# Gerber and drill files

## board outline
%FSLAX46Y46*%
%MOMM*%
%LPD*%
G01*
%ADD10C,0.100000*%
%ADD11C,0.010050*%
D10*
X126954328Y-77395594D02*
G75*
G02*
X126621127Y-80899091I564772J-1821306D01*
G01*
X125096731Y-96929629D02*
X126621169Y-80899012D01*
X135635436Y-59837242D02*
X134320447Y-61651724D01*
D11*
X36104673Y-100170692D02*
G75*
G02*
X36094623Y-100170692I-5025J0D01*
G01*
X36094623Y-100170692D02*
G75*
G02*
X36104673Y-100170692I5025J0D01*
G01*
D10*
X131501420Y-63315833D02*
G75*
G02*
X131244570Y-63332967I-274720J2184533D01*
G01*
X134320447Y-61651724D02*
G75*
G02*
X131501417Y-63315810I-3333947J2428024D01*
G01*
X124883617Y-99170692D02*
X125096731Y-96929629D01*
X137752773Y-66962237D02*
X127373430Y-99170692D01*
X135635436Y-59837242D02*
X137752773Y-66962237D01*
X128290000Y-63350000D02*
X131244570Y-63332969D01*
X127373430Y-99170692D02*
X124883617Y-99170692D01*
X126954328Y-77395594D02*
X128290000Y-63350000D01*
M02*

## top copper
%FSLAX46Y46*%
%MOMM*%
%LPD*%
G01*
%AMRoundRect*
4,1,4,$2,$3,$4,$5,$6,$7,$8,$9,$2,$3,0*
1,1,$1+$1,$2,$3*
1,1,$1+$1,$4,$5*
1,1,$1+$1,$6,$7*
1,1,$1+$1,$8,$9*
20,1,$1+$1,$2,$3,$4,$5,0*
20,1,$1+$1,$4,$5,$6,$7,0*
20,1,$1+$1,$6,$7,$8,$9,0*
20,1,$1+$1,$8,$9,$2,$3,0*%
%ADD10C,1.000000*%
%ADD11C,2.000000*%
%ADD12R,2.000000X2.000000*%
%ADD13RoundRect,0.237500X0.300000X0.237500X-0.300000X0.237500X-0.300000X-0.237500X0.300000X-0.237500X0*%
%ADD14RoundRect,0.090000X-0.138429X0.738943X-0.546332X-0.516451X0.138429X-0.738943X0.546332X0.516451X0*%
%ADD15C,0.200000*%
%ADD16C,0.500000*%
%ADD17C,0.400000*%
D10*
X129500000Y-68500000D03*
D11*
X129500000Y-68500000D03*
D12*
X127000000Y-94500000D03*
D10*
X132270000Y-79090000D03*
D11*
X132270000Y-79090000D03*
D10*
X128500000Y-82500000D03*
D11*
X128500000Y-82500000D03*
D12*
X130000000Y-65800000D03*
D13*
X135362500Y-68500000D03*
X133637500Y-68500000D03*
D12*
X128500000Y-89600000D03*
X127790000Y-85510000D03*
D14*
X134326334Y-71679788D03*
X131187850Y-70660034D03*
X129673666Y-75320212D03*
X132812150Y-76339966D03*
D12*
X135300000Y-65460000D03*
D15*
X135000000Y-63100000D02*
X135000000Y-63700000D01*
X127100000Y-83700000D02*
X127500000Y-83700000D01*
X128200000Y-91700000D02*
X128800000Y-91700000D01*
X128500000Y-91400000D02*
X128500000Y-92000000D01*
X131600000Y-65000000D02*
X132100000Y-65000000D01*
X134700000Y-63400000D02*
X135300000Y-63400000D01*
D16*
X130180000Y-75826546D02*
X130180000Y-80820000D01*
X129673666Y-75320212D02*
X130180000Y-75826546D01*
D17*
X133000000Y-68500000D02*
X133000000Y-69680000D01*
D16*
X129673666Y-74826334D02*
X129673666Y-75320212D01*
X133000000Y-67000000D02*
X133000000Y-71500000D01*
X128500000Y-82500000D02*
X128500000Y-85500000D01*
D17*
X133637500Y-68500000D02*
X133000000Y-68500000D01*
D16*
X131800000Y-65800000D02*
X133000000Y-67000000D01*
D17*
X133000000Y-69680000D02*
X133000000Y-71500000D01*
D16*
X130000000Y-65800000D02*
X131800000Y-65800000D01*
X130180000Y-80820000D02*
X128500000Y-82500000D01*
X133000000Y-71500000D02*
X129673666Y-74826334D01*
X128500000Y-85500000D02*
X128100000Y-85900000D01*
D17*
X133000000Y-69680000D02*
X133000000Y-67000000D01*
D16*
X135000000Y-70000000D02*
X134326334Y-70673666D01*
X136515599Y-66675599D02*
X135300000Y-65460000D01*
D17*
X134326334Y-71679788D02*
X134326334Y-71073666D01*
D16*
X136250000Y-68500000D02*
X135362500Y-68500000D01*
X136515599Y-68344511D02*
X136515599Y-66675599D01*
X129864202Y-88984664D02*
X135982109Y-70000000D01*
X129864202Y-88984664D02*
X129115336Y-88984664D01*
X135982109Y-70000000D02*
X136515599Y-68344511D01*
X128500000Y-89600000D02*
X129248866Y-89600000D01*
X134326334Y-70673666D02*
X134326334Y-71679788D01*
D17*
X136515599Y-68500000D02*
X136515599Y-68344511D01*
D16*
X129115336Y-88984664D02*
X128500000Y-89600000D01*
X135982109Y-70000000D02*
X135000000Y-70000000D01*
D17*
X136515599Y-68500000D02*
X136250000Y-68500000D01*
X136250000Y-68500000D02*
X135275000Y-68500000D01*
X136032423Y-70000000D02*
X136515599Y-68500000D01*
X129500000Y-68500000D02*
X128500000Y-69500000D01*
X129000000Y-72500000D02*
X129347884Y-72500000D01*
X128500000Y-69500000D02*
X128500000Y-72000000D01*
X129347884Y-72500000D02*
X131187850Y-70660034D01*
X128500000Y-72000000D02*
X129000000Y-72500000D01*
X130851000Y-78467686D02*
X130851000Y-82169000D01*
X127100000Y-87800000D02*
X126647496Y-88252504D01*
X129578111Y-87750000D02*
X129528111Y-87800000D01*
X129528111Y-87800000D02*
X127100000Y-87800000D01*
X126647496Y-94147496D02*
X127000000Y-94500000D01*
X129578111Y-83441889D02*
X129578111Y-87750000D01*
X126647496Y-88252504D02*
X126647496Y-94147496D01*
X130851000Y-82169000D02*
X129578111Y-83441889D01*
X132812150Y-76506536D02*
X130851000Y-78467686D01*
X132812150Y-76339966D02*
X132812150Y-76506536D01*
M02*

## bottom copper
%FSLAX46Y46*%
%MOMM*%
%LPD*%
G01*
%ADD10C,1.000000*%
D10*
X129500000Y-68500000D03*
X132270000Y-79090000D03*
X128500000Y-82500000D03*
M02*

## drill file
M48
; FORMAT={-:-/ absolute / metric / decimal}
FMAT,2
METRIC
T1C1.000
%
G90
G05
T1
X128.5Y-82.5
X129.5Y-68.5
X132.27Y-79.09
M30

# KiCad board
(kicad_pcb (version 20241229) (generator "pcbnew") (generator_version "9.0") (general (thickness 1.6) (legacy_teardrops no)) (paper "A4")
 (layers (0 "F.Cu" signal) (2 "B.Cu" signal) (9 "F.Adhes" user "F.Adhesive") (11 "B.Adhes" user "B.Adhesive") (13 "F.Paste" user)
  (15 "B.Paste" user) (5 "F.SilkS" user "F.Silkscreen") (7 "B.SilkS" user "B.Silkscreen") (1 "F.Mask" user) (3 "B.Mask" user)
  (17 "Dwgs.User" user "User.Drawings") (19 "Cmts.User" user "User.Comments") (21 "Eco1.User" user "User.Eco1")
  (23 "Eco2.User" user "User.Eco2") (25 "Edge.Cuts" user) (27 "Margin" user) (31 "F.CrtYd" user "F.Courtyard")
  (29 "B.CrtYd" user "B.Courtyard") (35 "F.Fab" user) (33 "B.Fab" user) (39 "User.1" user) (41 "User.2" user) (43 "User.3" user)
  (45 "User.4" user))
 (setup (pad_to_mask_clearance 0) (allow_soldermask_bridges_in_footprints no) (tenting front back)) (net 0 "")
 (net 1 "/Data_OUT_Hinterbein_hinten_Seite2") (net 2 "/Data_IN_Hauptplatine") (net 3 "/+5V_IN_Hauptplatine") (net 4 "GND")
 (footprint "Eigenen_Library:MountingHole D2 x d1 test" (layer "F.Cu") (at 129.5 68.5)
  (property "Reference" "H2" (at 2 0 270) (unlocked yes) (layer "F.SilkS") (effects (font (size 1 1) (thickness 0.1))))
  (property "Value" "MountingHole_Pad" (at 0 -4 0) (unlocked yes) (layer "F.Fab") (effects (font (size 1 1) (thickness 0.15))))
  (pad "1" thru_hole circle (at 0 0) (size 1 1) (drill 1) (layers "*.Cu" "*.Mask") (remove_unused_layers no)
   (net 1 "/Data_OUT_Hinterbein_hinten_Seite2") (zone_connect 2))
  (pad "1" connect circle (at 0 0) (size 2 2) (layers "F.Cu" "F.Mask") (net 1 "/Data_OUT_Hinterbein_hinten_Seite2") (zone_connect 2)))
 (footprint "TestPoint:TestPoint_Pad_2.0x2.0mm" (layer "F.Cu") (at 127 94.5)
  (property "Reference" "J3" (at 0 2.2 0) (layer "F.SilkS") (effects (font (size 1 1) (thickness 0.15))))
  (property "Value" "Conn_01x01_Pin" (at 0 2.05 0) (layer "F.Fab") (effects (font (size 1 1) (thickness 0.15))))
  (pad "1" smd rect (at 0 0) (size 2 2) (layers "F.Cu" "F.Mask") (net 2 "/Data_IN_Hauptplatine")))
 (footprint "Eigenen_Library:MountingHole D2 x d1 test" (layer "F.Cu") (at 132.27 79.09)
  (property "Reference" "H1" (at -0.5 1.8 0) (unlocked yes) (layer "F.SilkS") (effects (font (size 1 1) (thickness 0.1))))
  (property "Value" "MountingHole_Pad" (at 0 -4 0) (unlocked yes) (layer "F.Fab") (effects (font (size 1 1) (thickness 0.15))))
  (pad "1" thru_hole circle (at 0 0) (size 1 1) (drill 1) (layers "*.Cu" "*.Mask") (remove_unused_layers no) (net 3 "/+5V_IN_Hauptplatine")
   (zone_connect 2))
  (pad "1" connect circle (at 0 0) (size 2 2) (layers "F.Cu" "F.Mask") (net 3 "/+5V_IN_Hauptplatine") (zone_connect 2)))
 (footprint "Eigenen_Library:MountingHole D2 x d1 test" (layer "F.Cu") (at 128.5 82.5)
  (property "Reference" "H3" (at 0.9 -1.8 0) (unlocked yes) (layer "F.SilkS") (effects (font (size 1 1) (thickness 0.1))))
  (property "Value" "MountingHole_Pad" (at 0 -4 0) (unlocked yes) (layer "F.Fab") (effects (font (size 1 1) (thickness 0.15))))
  (pad "1" thru_hole circle (at 0 0) (size 1 1) (drill 1) (layers "*.Cu" "*.Mask") (remove_unused_layers no) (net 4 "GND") (zone_connect 2))
  (pad "1" connect circle (at 0 0) (size 2 2) (layers "F.Cu" "F.Mask") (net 4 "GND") (zone_connect 2)))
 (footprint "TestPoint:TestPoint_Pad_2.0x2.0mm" (layer "F.Cu") (at 130 65.8)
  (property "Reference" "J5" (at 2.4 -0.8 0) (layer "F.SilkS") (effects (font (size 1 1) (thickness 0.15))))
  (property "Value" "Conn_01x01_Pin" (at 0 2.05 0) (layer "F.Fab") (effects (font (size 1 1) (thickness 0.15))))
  (pad "1" smd rect (at 0 0) (size 2 2) (layers "F.Cu" "F.Mask") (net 4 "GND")))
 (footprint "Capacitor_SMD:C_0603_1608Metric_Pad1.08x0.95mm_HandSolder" (layer "F.Cu") (at 134.5 68.5 180)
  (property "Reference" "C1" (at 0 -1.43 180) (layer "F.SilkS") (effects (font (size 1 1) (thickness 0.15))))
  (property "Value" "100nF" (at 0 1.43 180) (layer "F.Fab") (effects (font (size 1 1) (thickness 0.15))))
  (pad "1" smd roundrect (at -0.8625 0 180) (size 1.075 0.95) (layers "F.Cu" "F.Mask" "F.Paste") (roundrect_rratio 0.25)
   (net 3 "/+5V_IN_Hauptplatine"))
  (pad "2" smd roundrect (at 0.8625 0 180) (size 1.075 0.95) (layers "F.Cu" "F.Mask" "F.Paste") (roundrect_rratio 0.25) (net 4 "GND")))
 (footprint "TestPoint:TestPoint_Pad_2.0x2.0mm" (layer "F.Cu") (at 128.5 89.6)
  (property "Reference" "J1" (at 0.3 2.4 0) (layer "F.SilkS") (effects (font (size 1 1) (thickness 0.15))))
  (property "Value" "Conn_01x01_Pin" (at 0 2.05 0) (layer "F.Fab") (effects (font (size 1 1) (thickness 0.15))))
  (pad "1" smd rect (at 0 0) (size 2 2) (layers "F.Cu" "F.Mask") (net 3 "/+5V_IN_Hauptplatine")))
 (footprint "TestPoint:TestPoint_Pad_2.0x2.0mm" (layer "F.Cu") (at 127.79 85.51)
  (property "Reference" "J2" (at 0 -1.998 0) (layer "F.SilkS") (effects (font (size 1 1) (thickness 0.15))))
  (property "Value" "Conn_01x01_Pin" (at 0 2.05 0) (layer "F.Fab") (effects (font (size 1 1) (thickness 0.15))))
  (pad "1" smd rect (at 0 0) (size 2 2) (layers "F.Cu" "F.Mask") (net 4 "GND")))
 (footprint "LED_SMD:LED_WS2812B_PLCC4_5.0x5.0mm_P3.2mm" (layer "F.Cu") (at 132 73.5 -108)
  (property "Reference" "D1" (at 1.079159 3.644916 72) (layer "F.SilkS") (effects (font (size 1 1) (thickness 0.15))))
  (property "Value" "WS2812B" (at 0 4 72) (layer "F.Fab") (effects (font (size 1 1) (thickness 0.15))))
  (pad "1" smd roundrect (at -2.450001 -1.649999 252) (size 1.5 0.9) (layers "F.Cu" "F.Mask" "F.Paste") (roundrect_rratio 0.1)
   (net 3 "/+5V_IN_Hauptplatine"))
  (pad "2" smd roundrect (at -2.45 1.649998 252) (size 1.5 0.9) (layers "F.Cu" "F.Mask" "F.Paste") (roundrect_rratio 0.1)
   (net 1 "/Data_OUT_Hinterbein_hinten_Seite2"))
  (pad "3" smd roundrect (at 2.450001 1.649999 252) (size 1.5 0.9) (layers "F.Cu" "F.Mask" "F.Paste") (roundrect_rratio 0.1) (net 4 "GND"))
  (pad "4" smd roundrect (at 2.45 -1.649998 252) (size 1.5 0.9) (layers "F.Cu" "F.Mask" "F.Paste") (roundrect_rratio 0.1)
   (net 2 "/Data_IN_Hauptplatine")))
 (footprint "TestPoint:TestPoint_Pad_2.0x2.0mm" (layer "F.Cu") (at 135.3 65.46)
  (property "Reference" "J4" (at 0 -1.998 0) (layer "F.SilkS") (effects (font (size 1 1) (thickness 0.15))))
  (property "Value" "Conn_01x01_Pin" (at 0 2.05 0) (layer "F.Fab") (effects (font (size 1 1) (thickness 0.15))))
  (pad "1" smd rect (at 0 0) (size 2 2) (layers "F.Cu" "F.Mask") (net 3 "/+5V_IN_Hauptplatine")))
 (gr_arc (start 126.954328 77.395594) (mid 129.417363 79.397367) (end 126.621169 80.899012) (stroke (width 0.1) (type default)) (locked yes)
  (layer "Edge.Cuts"))
 (gr_line (start 125.096731 96.929629) (end 126.621169 80.899012) (stroke (width 0.1) (type default)) (locked yes) (layer "Edge.Cuts"))
 (gr_line (start 135.635436 59.837242) (end 134.320447 61.651724) (stroke (width 0.1) (type default)) (locked yes) (layer "Edge.Cuts"))
 (gr_circle (center 36.099648 100.170692) (end 36.109648 100.170692) (stroke (width 0.0001) (type default)) (fill yes) (locked yes)
  (layer "Edge.Cuts"))
 (gr_arc (start 131.50142 63.315833) (mid 131.373246 63.328158) (end 131.24457 63.332969) (stroke (width 0.1) (type default)) (locked yes)
  (layer "Edge.Cuts"))
 (gr_arc (start 134.320447 61.651724) (mid 133.083107 62.775433) (end 131.50142 63.315833) (stroke (width 0.1) (type default)) (locked yes)
  (layer "Edge.Cuts"))
 (gr_line (start 124.883617 99.170692) (end 125.096731 96.929629) (stroke (width 0.1) (type default)) (locked yes) (layer "Edge.Cuts"))
 (gr_line (start 137.752773 66.962237) (end 127.37343 99.170692) (stroke (width 0.1) (type default)) (locked yes) (layer "Edge.Cuts"))
 (gr_line (start 135.635436 59.837242) (end 137.752773 66.962237) (stroke (width 0.1) (type default)) (locked yes) (layer "Edge.Cuts"))
 (gr_line (start 128.29 63.35) (end 131.24457 63.332969) (stroke (width 0.1) (type default)) (locked yes) (layer "Edge.Cuts"))
 (gr_line (start 127.37343 99.170692) (end 124.883617 99.170692) (stroke (width 0.1) (type default)) (locked yes) (layer "Edge.Cuts"))
 (gr_line (start 126.954328 77.395594) (end 128.29 63.35) (stroke (width 0.1) (type default)) (locked yes) (layer "Edge.Cuts"))
 (segment (start 135 63.1) (end 135 63.7) (width 0.2) (layer "F.Cu") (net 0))
 (segment (start 127.1 83.7) (end 127.5 83.7) (width 0.2) (layer "F.Cu") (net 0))
 (segment (start 128.2 91.7) (end 128.8 91.7) (width 0.2) (layer "F.Cu") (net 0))
 (segment (start 128.5 91.4) (end 128.5 92) (width 0.2) (layer "F.Cu") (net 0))
 (segment (start 131.6 65) (end 132.1 65) (width 0.2) (layer "F.Cu") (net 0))
 (segment (start 134.7 63.4) (end 135.3 63.4) (width 0.2) (layer "F.Cu") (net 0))
 (segment (start 130.18 75.826546) (end 130.18 80.82) (width 0.5) (layer "F.Cu") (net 4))
 (segment (start 129.673666 75.320212) (end 130.18 75.826546) (width 0.5) (layer "F.Cu") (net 4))
 (segment (start 133 68.5) (end 133 69.68) (width 0.4) (layer "F.Cu") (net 4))
 (segment (start 129.673666 74.826334) (end 129.673666 75.320212) (width 0.5) (layer "F.Cu") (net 4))
 (segment (start 133 67) (end 133 71.5) (width 0.5) (layer "F.Cu") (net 4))
 (segment (start 128.5 82.5) (end 128.5 85.5) (width 0.5) (layer "F.Cu") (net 4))
 (segment (start 133.6375 68.5) (end 133 68.5) (width 0.4) (layer "F.Cu") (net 4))
 (segment (start 131.8 65.8) (end 133 67) (width 0.5) (layer "F.Cu") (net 4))
 (segment (start 133 69.68) (end 133 71.5) (width 0.4) (layer "F.Cu") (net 4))
 (segment (start 130 65.8) (end 131.8 65.8) (width 0.5) (layer "F.Cu") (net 4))
 (segment (start 130.18 80.82) (end 128.5 82.5) (width 0.5) (layer "F.Cu") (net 4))
 (segment (start 133 71.5) (end 129.673666 74.826334) (width 0.5) (layer "F.Cu") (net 4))
 (segment (start 128.5 85.5) (end 128.1 85.9) (width 0.5) (layer "F.Cu") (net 4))
 (segment (start 133 69.68) (end 133 67) (width 0.4) (layer "F.Cu") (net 4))
 (segment (start 135 70) (end 134.326334 70.673666) (width 0.5) (layer "F.Cu") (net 3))
 (segment (start 136.515599 66.675599) (end 135.3 65.46) (width 0.5) (layer "F.Cu") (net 3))
 (segment (start 134.326334 71.679788) (end 134.326334 71.073666) (width 0.4) (layer "F.Cu") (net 3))
 (segment (start 136.25 68.5) (end 135.3625 68.5) (width 0.5) (layer "F.Cu") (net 3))
 (segment (start 136.515599 68.344511) (end 136.515599 66.675599) (width 0.5) (layer "F.Cu") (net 3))
 (segment (start 129.864202 88.984664) (end 135.982109 70) (width 0.5) (layer "F.Cu") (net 3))
 (segment (start 129.864202 88.984664) (end 129.115336 88.984664) (width 0.5) (layer "F.Cu") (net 3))
 (segment (start 135.982109 70) (end 136.515599 68.344511) (width 0.5) (layer "F.Cu") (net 3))
 (segment (start 128.5 89.6) (end 129.248866 89.6) (width 0.5) (layer "F.Cu") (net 3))
 (segment (start 134.326334 70.673666) (end 134.326334 71.679788) (width 0.5) (layer "F.Cu") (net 3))
 (segment (start 136.515599 68.5) (end 136.515599 68.344511) (width 0.4) (layer "F.Cu") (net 3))
 (segment (start 129.115336 88.984664) (end 128.5 89.6) (width 0.5) (layer "F.Cu") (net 3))
 (segment (start 135.982109 70) (end 135 70) (width 0.5) (layer "F.Cu") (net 3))
 (segment (start 136.515599 68.5) (end 136.25 68.5) (width 0.4) (layer "F.Cu") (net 3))
 (segment (start 136.25 68.5) (end 135.275 68.5) (width 0.4) (layer "F.Cu") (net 3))
 (segment (start 136.032423 70) (end 136.515599 68.5) (width 0.4) (layer "F.Cu") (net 3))
 (segment (start 129.5 68.5) (end 128.5 69.5) (width 0.4) (layer "F.Cu") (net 1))
 (segment (start 129 72.5) (end 129.347884 72.5) (width 0.4) (layer "F.Cu") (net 1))
 (segment (start 128.5 69.5) (end 128.5 72) (width 0.4) (layer "F.Cu") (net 1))
 (segment (start 129.347884 72.5) (end 131.18785 70.660034) (width 0.4) (layer "F.Cu") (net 1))
 (segment (start 128.5 72) (end 129 72.5) (width 0.4) (layer "F.Cu") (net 1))
 (segment (start 130.851 78.467686) (end 130.851 82.169) (width 0.4) (layer "F.Cu") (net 2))
 (segment (start 127.1 87.8) (end 126.647496 88.252504) (width 0.4) (layer "F.Cu") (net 2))
 (segment (start 129.578111 87.75) (end 129.528111 87.8) (width 0.4) (layer "F.Cu") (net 2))
 (segment (start 129.528111 87.8) (end 127.1 87.8) (width 0.4) (layer "F.Cu") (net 2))
 (segment (start 126.647496 94.147496) (end 127 94.5) (width 0.4) (layer "F.Cu") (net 2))
 (segment (start 129.578111 83.441889) (end 129.578111 87.75) (width 0.4) (layer "F.Cu") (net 2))
 (segment (start 126.647496 88.252504) (end 126.647496 94.147496) (width 0.4) (layer "F.Cu") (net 2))
 (segment (start 130.851 82.169) (end 129.578111 83.441889) (width 0.4) (layer "F.Cu") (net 2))
 (segment (start 132.81215 76.506536) (end 130.851 78.467686) (width 0.4) (layer "F.Cu") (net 2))
 (segment (start 132.81215 76.339966) (end 132.81215 76.506536) (width 0.4) (layer "F.Cu") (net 2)))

